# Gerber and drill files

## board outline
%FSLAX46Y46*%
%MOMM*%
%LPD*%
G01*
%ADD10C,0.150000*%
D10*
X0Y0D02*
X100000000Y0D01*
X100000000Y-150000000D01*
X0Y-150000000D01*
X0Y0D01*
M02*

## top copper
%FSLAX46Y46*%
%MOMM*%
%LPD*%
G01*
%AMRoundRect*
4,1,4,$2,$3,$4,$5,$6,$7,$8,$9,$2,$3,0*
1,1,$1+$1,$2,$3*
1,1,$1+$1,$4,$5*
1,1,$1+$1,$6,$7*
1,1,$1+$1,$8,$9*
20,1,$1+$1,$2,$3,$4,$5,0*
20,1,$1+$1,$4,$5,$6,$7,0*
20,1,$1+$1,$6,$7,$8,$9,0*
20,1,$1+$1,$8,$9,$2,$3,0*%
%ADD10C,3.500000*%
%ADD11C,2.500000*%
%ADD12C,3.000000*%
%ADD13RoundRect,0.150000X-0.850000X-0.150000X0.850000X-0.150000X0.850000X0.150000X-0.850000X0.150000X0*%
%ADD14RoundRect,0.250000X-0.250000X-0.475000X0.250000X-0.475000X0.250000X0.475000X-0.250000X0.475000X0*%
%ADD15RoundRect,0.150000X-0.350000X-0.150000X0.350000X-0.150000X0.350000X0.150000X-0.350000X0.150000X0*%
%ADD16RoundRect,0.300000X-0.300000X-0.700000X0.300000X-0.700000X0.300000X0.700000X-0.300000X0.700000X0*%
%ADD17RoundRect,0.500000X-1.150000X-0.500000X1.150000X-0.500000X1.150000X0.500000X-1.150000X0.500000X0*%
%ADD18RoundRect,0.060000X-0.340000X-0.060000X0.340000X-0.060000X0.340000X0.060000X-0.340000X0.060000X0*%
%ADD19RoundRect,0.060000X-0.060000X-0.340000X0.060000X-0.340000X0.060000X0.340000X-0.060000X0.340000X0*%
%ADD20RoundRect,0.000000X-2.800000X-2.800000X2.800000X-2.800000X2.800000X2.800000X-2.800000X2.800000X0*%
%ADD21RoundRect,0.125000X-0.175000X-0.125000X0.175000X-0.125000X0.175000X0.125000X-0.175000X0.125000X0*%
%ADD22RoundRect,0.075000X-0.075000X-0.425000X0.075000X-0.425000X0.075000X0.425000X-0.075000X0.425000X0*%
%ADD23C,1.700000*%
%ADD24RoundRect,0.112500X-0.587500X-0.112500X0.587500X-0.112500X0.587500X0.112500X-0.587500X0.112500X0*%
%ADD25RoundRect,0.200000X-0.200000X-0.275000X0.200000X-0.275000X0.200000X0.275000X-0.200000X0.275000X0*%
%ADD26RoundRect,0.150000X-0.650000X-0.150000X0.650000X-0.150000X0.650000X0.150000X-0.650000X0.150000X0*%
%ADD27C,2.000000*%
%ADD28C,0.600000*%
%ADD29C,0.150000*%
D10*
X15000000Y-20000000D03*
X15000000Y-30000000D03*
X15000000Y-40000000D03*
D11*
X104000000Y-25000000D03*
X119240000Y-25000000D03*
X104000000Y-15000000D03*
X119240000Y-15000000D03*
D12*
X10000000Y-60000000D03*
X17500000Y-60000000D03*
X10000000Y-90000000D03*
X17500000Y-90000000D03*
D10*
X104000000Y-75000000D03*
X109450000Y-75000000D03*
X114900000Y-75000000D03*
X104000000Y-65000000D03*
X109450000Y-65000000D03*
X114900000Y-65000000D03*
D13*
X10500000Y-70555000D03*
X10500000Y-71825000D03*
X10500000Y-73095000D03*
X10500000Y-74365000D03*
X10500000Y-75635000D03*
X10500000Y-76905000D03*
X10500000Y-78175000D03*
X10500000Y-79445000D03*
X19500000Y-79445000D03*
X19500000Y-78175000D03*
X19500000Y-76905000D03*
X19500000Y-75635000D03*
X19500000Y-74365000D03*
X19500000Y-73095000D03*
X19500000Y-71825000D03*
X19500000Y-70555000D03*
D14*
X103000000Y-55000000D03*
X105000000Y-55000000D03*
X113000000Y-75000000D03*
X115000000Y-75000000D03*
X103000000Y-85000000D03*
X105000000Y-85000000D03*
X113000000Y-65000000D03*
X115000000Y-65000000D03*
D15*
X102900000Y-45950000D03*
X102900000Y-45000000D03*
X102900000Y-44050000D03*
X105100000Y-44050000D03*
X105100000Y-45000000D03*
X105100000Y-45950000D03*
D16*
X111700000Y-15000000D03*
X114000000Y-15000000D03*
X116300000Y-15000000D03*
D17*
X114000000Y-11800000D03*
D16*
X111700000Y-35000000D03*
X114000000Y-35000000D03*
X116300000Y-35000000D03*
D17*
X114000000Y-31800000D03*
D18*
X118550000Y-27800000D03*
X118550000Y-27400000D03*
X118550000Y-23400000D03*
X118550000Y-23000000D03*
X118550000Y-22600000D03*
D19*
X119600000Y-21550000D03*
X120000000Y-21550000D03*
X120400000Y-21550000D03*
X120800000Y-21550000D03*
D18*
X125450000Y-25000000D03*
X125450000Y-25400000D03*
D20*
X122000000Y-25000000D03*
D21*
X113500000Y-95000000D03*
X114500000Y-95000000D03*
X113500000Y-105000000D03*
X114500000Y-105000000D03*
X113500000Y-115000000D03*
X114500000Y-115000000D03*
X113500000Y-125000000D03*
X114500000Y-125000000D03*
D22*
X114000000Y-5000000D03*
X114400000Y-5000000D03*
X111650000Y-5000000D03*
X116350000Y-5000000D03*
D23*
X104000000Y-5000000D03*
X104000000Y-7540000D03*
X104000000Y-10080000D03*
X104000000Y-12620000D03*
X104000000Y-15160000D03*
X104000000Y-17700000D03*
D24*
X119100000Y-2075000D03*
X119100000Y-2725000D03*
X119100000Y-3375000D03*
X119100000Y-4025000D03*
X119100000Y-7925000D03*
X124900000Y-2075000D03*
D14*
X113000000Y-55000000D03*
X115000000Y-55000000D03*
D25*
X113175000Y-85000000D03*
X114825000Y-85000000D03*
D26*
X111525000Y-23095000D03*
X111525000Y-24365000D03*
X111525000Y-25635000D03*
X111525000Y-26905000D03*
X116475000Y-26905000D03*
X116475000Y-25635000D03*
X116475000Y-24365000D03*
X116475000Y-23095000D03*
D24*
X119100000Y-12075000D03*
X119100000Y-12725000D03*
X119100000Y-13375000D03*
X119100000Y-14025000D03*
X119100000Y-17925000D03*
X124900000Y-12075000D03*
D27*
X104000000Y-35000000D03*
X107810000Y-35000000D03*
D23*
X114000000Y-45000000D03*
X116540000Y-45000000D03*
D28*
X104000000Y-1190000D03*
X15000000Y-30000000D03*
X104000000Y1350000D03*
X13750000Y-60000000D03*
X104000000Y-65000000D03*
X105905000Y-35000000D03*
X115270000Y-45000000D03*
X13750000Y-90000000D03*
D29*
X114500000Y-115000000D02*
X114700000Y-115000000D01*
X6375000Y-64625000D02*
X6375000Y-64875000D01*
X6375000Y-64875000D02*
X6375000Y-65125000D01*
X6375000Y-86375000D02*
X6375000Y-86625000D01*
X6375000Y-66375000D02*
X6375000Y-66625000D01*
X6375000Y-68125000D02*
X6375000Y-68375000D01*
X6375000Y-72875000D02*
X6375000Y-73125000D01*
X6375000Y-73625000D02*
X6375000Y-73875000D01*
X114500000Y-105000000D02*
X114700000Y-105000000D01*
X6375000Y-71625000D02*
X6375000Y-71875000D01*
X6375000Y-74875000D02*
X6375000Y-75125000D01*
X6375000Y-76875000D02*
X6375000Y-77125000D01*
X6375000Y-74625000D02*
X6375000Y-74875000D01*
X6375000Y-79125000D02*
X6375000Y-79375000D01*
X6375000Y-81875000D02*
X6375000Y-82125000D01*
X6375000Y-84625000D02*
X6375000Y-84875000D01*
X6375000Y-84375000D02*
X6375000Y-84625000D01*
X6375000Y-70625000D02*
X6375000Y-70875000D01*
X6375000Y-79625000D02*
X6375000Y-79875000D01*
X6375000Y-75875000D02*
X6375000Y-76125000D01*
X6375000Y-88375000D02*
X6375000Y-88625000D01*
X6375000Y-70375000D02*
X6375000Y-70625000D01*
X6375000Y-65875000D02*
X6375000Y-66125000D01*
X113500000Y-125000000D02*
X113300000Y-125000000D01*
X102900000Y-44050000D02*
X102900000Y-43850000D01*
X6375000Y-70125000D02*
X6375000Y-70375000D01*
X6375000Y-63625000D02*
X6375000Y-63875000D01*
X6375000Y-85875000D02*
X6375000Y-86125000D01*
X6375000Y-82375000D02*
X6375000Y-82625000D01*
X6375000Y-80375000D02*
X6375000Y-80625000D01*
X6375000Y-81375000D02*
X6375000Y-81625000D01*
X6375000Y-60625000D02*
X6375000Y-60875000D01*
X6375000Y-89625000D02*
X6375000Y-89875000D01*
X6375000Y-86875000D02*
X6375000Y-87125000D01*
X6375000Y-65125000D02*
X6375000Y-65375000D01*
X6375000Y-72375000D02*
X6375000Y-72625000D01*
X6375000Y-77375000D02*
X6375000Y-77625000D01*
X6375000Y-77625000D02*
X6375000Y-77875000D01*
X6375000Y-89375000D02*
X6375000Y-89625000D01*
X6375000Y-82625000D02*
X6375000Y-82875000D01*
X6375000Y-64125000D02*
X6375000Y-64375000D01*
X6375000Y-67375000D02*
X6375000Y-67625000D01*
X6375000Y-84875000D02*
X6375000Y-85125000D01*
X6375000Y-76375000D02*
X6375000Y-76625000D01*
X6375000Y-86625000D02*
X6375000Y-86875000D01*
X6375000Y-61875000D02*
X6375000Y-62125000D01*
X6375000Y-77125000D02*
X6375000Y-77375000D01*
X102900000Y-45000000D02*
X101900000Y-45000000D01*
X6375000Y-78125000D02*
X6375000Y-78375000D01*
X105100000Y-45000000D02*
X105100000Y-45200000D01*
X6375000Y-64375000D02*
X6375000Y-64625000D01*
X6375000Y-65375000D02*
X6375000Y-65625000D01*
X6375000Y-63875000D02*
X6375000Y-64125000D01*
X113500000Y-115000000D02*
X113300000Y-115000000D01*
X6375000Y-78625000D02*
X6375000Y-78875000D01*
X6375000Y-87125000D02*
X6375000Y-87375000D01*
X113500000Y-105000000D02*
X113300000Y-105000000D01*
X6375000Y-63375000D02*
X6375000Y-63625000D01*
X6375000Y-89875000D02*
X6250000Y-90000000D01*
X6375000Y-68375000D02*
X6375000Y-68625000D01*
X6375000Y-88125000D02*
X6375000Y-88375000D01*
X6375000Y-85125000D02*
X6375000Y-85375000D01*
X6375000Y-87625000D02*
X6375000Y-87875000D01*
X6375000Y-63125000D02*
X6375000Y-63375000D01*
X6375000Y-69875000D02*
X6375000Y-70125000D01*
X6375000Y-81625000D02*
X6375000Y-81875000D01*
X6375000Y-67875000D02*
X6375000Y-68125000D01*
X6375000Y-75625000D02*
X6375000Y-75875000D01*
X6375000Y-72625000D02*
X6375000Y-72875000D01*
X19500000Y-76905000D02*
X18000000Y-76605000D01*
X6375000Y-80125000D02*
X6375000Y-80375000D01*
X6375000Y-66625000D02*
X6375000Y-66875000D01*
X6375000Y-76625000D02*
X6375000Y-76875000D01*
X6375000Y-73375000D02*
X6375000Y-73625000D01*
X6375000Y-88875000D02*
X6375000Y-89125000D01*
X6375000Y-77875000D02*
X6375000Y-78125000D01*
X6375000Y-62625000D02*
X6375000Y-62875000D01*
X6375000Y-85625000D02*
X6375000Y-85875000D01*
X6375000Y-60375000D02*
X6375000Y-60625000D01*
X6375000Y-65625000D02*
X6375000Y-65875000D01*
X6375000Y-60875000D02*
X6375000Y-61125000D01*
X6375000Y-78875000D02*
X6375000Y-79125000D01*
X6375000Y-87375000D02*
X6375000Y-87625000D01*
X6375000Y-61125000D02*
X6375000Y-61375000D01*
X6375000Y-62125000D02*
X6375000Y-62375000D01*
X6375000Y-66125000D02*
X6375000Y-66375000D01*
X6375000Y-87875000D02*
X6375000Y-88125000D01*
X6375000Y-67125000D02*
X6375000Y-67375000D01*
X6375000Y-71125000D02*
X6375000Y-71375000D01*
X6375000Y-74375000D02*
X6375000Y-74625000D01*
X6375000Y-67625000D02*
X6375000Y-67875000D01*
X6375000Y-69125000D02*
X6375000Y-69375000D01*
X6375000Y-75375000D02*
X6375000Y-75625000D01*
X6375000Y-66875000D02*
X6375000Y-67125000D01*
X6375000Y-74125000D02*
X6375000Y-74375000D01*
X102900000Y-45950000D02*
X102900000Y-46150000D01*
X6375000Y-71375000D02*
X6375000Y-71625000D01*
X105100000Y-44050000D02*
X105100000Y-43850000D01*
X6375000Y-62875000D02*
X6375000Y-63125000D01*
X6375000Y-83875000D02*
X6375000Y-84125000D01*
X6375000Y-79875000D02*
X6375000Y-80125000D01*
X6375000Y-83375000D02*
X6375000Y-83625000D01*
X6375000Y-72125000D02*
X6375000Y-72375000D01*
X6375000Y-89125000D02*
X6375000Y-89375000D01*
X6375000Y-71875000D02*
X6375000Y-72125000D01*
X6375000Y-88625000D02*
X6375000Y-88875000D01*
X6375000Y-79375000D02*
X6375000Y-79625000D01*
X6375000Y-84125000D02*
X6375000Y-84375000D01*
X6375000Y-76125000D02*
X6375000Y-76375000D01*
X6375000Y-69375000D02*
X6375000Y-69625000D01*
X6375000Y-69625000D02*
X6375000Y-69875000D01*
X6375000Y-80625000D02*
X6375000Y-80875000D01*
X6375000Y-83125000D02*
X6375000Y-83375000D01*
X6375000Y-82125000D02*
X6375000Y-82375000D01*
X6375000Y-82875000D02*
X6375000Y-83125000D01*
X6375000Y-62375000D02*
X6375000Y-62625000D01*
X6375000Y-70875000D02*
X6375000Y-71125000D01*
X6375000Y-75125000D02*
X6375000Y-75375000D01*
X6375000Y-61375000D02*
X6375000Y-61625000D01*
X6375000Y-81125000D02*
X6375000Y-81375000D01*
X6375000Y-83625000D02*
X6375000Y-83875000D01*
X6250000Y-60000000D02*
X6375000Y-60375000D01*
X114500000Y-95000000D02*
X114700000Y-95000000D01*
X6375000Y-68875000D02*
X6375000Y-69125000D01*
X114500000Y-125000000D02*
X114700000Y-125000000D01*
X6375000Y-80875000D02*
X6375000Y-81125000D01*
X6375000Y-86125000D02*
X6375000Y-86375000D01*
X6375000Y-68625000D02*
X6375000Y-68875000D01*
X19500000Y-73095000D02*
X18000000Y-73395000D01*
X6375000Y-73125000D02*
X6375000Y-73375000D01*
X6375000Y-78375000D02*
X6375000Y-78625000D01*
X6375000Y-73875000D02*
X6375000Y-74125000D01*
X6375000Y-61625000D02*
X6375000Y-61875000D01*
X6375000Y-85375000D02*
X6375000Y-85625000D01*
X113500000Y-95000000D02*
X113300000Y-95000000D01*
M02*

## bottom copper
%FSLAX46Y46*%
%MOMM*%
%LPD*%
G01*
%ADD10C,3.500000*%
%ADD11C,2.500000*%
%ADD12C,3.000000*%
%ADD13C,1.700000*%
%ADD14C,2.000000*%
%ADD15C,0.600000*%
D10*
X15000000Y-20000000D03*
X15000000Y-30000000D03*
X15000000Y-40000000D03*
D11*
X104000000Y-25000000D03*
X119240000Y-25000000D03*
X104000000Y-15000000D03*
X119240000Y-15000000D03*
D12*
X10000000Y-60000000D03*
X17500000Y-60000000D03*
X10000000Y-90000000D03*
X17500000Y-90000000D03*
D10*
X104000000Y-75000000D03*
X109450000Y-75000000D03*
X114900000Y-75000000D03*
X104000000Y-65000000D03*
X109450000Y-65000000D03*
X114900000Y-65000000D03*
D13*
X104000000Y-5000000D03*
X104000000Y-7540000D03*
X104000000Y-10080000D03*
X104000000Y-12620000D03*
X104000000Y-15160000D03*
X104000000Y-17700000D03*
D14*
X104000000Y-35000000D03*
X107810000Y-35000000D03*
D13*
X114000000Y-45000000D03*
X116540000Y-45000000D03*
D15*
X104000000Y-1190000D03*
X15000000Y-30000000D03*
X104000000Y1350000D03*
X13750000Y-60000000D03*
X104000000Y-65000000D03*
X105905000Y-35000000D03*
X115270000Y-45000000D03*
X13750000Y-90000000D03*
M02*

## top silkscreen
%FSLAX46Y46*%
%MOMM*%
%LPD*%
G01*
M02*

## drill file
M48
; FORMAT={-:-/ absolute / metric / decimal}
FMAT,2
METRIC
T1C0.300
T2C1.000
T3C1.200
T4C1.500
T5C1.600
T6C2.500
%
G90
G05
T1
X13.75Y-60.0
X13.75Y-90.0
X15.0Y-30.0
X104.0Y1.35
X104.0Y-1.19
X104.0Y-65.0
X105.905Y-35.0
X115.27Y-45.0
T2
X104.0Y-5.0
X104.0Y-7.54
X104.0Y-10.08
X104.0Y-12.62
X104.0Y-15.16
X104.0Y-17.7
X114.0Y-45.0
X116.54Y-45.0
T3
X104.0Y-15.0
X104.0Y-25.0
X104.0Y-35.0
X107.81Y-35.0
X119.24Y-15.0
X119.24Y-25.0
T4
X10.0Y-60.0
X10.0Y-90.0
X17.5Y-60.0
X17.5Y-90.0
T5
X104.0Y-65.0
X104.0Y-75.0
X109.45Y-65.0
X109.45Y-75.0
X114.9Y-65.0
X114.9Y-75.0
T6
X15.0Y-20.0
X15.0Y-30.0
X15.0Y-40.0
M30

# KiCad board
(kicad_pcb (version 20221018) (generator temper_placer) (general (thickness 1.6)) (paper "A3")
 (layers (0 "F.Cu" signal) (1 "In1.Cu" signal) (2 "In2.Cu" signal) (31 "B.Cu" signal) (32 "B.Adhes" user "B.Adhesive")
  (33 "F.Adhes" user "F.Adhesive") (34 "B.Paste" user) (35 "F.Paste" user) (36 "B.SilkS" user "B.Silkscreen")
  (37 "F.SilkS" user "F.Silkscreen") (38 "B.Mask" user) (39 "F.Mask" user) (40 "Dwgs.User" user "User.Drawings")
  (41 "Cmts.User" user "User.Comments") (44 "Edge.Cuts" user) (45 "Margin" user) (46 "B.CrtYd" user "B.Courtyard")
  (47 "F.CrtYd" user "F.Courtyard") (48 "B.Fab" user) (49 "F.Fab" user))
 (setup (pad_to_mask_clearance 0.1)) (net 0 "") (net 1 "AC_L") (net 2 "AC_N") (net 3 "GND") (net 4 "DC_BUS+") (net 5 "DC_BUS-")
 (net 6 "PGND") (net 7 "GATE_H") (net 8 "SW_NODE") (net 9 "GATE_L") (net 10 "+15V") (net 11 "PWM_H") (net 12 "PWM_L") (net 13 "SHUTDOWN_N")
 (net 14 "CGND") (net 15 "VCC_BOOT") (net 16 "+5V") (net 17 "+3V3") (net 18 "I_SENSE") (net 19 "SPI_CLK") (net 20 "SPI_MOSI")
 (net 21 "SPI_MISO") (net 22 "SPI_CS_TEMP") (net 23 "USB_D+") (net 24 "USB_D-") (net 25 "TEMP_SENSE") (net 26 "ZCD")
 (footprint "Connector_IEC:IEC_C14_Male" (layer "F.Cu") (at 15 20 0) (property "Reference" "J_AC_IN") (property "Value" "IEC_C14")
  (pad "1" thru_hole circle (at 0 0) (size 3.5 3.5) (drill 2.5) (layers *.Cu *.Mask) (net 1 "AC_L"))
  (pad "2" thru_hole circle (at 0 10) (size 3.5 3.5) (drill 2.5) (layers *.Cu *.Mask) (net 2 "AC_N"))
  (pad "3" thru_hole circle (at 0 20) (size 3.5 3.5) (drill 2.5) (layers *.Cu *.Mask) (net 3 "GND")))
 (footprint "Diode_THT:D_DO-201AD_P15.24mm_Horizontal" (layer "F.Cu") (at 104 25 0) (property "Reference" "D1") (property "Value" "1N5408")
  (pad "1" thru_hole circle (at 0 0) (size 2.5 2.5) (drill 1.2) (layers *.Cu *.Mask) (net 1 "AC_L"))
  (pad "2" thru_hole circle (at 15.24 0) (size 2.5 2.5) (drill 1.2) (layers *.Cu *.Mask) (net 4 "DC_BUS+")))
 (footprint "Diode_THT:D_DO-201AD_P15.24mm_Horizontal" (layer "F.Cu") (at 104 15 0) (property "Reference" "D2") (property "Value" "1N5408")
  (pad "1" thru_hole circle (at 0 0) (size 2.5 2.5) (drill 1.2) (layers *.Cu *.Mask) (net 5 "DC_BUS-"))
  (pad "2" thru_hole circle (at 15.24 0) (size 2.5 2.5) (drill 1.2) (layers *.Cu *.Mask) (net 2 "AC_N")))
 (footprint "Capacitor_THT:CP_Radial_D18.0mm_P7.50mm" (layer "F.Cu") (at 10 60 0) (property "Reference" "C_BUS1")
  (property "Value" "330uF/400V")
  (pad "1" thru_hole circle (at 0 0) (size 3 3) (drill 1.5) (layers *.Cu *.Mask) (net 4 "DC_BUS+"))
  (pad "2" thru_hole circle (at 7.5 0) (size 3 3) (drill 1.5) (layers *.Cu *.Mask) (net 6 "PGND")))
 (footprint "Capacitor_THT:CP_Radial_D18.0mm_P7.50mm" (layer "F.Cu") (at 10 90 0) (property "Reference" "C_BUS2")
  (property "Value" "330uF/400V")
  (pad "1" thru_hole circle (at 0 0) (size 3 3) (drill 1.5) (layers *.Cu *.Mask) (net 4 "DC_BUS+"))
  (pad "2" thru_hole circle (at 7.5 0) (size 3 3) (drill 1.5) (layers *.Cu *.Mask) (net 6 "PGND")))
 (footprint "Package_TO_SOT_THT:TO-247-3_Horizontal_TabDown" (layer "F.Cu") (at 104 75 0) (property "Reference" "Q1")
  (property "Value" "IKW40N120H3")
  (pad "1" thru_hole circle (at 0 0) (size 3.5 3.5) (drill 1.6) (layers *.Cu *.Mask) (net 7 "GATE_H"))
  (pad "2" thru_hole circle (at 5.45 0) (size 3.5 3.5) (drill 1.6) (layers *.Cu *.Mask) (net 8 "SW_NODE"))
  (pad "3" thru_hole circle (at 10.9 0) (size 3.5 3.5) (drill 1.6) (layers *.Cu *.Mask) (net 4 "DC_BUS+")))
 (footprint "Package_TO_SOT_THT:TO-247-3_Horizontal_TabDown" (layer "F.Cu") (at 104 65 0) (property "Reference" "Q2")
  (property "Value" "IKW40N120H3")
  (pad "1" thru_hole circle (at 0 0) (size 3.5 3.5) (drill 1.6) (layers *.Cu *.Mask) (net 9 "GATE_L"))
  (pad "2" thru_hole circle (at 5.45 0) (size 3.5 3.5) (drill 1.6) (layers *.Cu *.Mask) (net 6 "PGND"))
  (pad "3" thru_hole circle (at 10.9 0) (size 3.5 3.5) (drill 1.6) (layers *.Cu *.Mask) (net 8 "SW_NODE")))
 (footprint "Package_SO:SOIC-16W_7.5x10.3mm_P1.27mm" (layer "F.Cu") (at 15 75 0) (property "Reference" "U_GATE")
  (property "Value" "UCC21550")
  (pad "1" smd roundrect (at -4.5 -4.445) (size 2 0.6) (layers "F.Cu" "F.Paste" "F.Mask") (roundrect_rratio 0.25) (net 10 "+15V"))
  (pad "2" smd roundrect (at -4.5 -3.175) (size 2 0.6) (layers "F.Cu" "F.Paste" "F.Mask") (roundrect_rratio 0.25) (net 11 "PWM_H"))
  (pad "3" smd roundrect (at -4.5 -1.905) (size 2 0.6) (layers "F.Cu" "F.Paste" "F.Mask") (roundrect_rratio 0.25) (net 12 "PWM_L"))
  (pad "4" smd roundrect (at -4.5 -0.635) (size 2 0.6) (layers "F.Cu" "F.Paste" "F.Mask") (roundrect_rratio 0.25) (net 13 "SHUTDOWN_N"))
  (pad "5" smd roundrect (at -4.5 0.635) (size 2 0.6) (layers "F.Cu" "F.Paste" "F.Mask") (roundrect_rratio 0.25) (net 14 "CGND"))
  (pad "6" smd roundrect (at -4.5 1.905) (size 2 0.6) (layers "F.Cu" "F.Paste" "F.Mask") (roundrect_rratio 0.25) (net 14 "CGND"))
  (pad "7" smd roundrect (at -4.5 3.175) (size 2 0.6) (layers "F.Cu" "F.Paste" "F.Mask") (roundrect_rratio 0.25) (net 14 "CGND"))
  (pad "8" smd roundrect (at -4.5 4.445) (size 2 0.6) (layers "F.Cu" "F.Paste" "F.Mask") (roundrect_rratio 0.25) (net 14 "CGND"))
  (pad "9" smd roundrect (at 4.5 4.445) (size 2 0.6) (layers "F.Cu" "F.Paste" "F.Mask") (roundrect_rratio 0.25) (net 8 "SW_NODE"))
  (pad "10" smd roundrect (at 4.5 3.175) (size 2 0.6) (layers "F.Cu" "F.Paste" "F.Mask") (roundrect_rratio 0.25) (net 9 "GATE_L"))
  (pad "11" smd roundrect (at 4.5 1.905) (size 2 0.6) (layers "F.Cu" "F.Paste" "F.Mask") (roundrect_rratio 0.25) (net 10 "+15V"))
  (pad "12" smd roundrect (at 4.5 0.635) (size 2 0.6) (layers "F.Cu" "F.Paste" "F.Mask") (roundrect_rratio 0.25) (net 6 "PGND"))
  (pad "13" smd roundrect (at 4.5 -0.635) (size 2 0.6) (layers "F.Cu" "F.Paste" "F.Mask") (roundrect_rratio 0.25) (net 6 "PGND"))
  (pad "14" smd roundrect (at 4.5 -1.905) (size 2 0.6) (layers "F.Cu" "F.Paste" "F.Mask") (roundrect_rratio 0.25) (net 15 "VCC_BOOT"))
  (pad "15" smd roundrect (at 4.5 -3.175) (size 2 0.6) (layers "F.Cu" "F.Paste" "F.Mask") (roundrect_rratio 0.25) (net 7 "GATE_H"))
  (pad "16" smd roundrect (at 4.5 -4.445) (size 2 0.6) (layers "F.Cu" "F.Paste" "F.Mask") (roundrect_rratio 0.25) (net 8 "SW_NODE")))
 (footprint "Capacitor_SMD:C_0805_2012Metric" (layer "F.Cu") (at 104 55 0) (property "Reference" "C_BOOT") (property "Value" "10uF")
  (pad "1" smd roundrect (at -1 0) (size 1 1.45) (layers "F.Cu" "F.Paste" "F.Mask") (roundrect_rratio 0.25) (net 15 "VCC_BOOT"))
  (pad "2" smd roundrect (at 1 0) (size 1 1.45) (layers "F.Cu" "F.Paste" "F.Mask") (roundrect_rratio 0.25) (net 8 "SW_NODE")))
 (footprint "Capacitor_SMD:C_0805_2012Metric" (layer "F.Cu") (at 114 75 0) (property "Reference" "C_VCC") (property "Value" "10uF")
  (pad "1" smd roundrect (at -1 0) (size 1 1.45) (layers "F.Cu" "F.Paste" "F.Mask") (roundrect_rratio 0.25) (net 10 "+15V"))
  (pad "2" smd roundrect (at 1 0) (size 1 1.45) (layers "F.Cu" "F.Paste" "F.Mask") (roundrect_rratio 0.25) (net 14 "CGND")))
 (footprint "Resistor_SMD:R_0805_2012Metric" (layer "F.Cu") (at 104 85 0) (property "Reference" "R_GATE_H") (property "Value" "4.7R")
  (pad "1" smd roundrect (at -1 0) (size 1 1.45) (layers "F.Cu" "F.Paste" "F.Mask") (roundrect_rratio 0.25) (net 7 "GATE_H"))
  (pad "2" smd roundrect (at 1 0) (size 1 1.45) (layers "F.Cu" "F.Paste" "F.Mask") (roundrect_rratio 0.25) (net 7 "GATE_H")))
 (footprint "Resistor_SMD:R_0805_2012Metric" (layer "F.Cu") (at 114 65 0) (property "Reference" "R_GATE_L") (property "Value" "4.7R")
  (pad "1" smd roundrect (at -1 0) (size 1 1.45) (layers "F.Cu" "F.Paste" "F.Mask") (roundrect_rratio 0.25) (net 9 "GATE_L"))
  (pad "2" smd roundrect (at 1 0) (size 1 1.45) (layers "F.Cu" "F.Paste" "F.Mask") (roundrect_rratio 0.25) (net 9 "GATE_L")))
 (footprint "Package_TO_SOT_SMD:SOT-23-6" (layer "F.Cu") (at 104 45 0) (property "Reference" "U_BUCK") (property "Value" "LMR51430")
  (pad "1" smd roundrect (at -1.1 0.95) (size 1 0.6) (layers "F.Cu" "F.Paste" "F.Mask") (roundrect_rratio 0.25) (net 3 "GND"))
  (pad "2" smd roundrect (at -1.1 0) (size 1 0.6) (layers "F.Cu" "F.Paste" "F.Mask") (roundrect_rratio 0.25) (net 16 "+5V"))
  (pad "3" smd roundrect (at -1.1 -0.95) (size 1 0.6) (layers "F.Cu" "F.Paste" "F.Mask") (roundrect_rratio 0.25) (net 10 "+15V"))
  (pad "4" smd roundrect (at 1.1 -0.95) (size 1 0.6) (layers "F.Cu" "F.Paste" "F.Mask") (roundrect_rratio 0.25) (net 16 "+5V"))
  (pad "5" smd roundrect (at 1.1 0) (size 1 0.6) (layers "F.Cu" "F.Paste" "F.Mask") (roundrect_rratio 0.25) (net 3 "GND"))
  (pad "6" smd roundrect (at 1.1 0.95) (size 1 0.6) (layers "F.Cu" "F.Paste" "F.Mask") (roundrect_rratio 0.25) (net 3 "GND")))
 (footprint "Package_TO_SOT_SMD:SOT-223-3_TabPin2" (layer "F.Cu") (at 114 15 0) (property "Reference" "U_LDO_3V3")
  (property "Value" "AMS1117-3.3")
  (pad "1" smd roundrect (at -2.3 0) (size 1.2 2) (layers "F.Cu" "F.Paste" "F.Mask") (roundrect_rratio 0.25) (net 3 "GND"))
  (pad "2" smd roundrect (at 0 0) (size 1.2 2) (layers "F.Cu" "F.Paste" "F.Mask") (roundrect_rratio 0.25) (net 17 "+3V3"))
  (pad "3" smd roundrect (at 2.3 0) (size 1.2 2) (layers "F.Cu" "F.Paste" "F.Mask") (roundrect_rratio 0.25) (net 16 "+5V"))
  (pad "4" smd roundrect (at 0 -3.2) (size 3.3 2) (layers "F.Cu" "F.Paste" "F.Mask") (roundrect_rratio 0.25) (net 17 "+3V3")))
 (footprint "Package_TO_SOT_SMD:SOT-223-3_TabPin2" (layer "F.Cu") (at 114 35 0) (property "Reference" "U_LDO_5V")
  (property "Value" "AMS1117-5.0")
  (pad "1" smd roundrect (at -2.3 0) (size 1.2 2) (layers "F.Cu" "F.Paste" "F.Mask") (roundrect_rratio 0.25) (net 3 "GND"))
  (pad "2" smd roundrect (at 0 0) (size 1.2 2) (layers "F.Cu" "F.Paste" "F.Mask") (roundrect_rratio 0.25) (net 16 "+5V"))
  (pad "3" smd roundrect (at 2.3 0) (size 1.2 2) (layers "F.Cu" "F.Paste" "F.Mask") (roundrect_rratio 0.25) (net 10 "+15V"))
  (pad "4" smd roundrect (at 0 -3.2) (size 3.3 2) (layers "F.Cu" "F.Paste" "F.Mask") (roundrect_rratio 0.25) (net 16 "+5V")))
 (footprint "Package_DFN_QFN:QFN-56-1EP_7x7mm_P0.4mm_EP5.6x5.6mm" (layer "F.Cu") (at 122 25 0) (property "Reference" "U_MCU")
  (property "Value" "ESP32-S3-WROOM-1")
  (pad "1" smd roundrect (at -3.45 2.8) (size 0.8 0.24) (layers "F.Cu" "F.Paste" "F.Mask") (roundrect_rratio 0.25) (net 17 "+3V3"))
  (pad "2" smd roundrect (at -3.45 2.4) (size 0.8 0.24) (layers "F.Cu" "F.Paste" "F.Mask") (roundrect_rratio 0.25) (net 3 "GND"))
  (pad "13" smd roundrect (at -3.45 -1.6) (size 0.8 0.24) (layers "F.Cu" "F.Paste" "F.Mask") (roundrect_rratio 0.25) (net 11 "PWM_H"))
  (pad "14" smd roundrect (at -3.45 -2) (size 0.8 0.24) (layers "F.Cu" "F.Paste" "F.Mask") (roundrect_rratio 0.25) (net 12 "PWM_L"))
  (pad "15" smd roundrect (at -3.45 -2.4) (size 0.8 0.24) (layers "F.Cu" "F.Paste" "F.Mask") (roundrect_rratio 0.25) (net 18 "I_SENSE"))
  (pad "20" smd roundrect (at -2.4 -3.45) (size 0.24 0.8) (layers "F.Cu" "F.Paste" "F.Mask") (roundrect_rratio 0.25) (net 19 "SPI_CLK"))
  (pad "21" smd roundrect (at -2 -3.45) (size 0.24 0.8) (layers "F.Cu" "F.Paste" "F.Mask") (roundrect_rratio 0.25) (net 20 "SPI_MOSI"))
  (pad "22" smd roundrect (at -1.6 -3.45) (size 0.24 0.8) (layers "F.Cu" "F.Paste" "F.Mask") (roundrect_rratio 0.25) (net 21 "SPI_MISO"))
  (pad "23" smd roundrect (at -1.2 -3.45) (size 0.24 0.8) (layers "F.Cu" "F.Paste" "F.Mask") (roundrect_rratio 0.25) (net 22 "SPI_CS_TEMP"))
  (pad "40" smd roundrect (at 3.45 0) (size 0.8 0.24) (layers "F.Cu" "F.Paste" "F.Mask") (roundrect_rratio 0.25) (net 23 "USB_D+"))
  (pad "41" smd roundrect (at 3.45 0.4) (size 0.8 0.24) (layers "F.Cu" "F.Paste" "F.Mask") (roundrect_rratio 0.25) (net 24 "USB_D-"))
  (pad "57" smd roundrect (at 0 0) (size 5.6 5.6) (layers "F.Cu" "F.Paste" "F.Mask") (roundrect_rratio 0) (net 3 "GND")))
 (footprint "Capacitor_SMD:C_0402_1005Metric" (layer "F.Cu") (at 114 95 0) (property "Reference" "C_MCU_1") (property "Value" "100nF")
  (pad "1" smd roundrect (at -0.5 0) (size 0.6 0.5) (layers "F.Cu" "F.Paste" "F.Mask") (roundrect_rratio 0.25) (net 17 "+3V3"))
  (pad "2" smd roundrect (at 0.5 0) (size 0.6 0.5) (layers "F.Cu" "F.Paste" "F.Mask") (roundrect_rratio 0.25) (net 3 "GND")))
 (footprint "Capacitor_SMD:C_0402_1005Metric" (layer "F.Cu") (at 114 105 0) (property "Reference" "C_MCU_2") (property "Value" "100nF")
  (pad "1" smd roundrect (at -0.5 0) (size 0.6 0.5) (layers "F.Cu" "F.Paste" "F.Mask") (roundrect_rratio 0.25) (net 17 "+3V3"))
  (pad "2" smd roundrect (at 0.5 0) (size 0.6 0.5) (layers "F.Cu" "F.Paste" "F.Mask") (roundrect_rratio 0.25) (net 3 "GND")))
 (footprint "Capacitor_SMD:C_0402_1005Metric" (layer "F.Cu") (at 114 115 0) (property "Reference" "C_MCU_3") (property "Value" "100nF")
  (pad "1" smd roundrect (at -0.5 0) (size 0.6 0.5) (layers "F.Cu" "F.Paste" "F.Mask") (roundrect_rratio 0.25) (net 17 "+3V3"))
  (pad "2" smd roundrect (at 0.5 0) (size 0.6 0.5) (layers "F.Cu" "F.Paste" "F.Mask") (roundrect_rratio 0.25) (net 3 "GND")))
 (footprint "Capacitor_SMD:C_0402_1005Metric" (layer "F.Cu") (at 114 125 0) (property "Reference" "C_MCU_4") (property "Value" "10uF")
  (pad "1" smd roundrect (at -0.5 0) (size 0.6 0.5) (layers "F.Cu" "F.Paste" "F.Mask") (roundrect_rratio 0.25) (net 17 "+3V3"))
  (pad "2" smd roundrect (at 0.5 0) (size 0.6 0.5) (layers "F.Cu" "F.Paste" "F.Mask") (roundrect_rratio 0.25) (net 3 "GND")))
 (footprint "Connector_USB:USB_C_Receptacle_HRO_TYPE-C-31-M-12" (layer "F.Cu") (at 114 5 0) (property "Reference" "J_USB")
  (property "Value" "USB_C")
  (pad "A6" smd roundrect (at 0 0) (size 0.3 1) (layers "F.Cu" "F.Paste" "F.Mask") (roundrect_rratio 0.25) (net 23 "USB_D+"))
  (pad "B6" smd roundrect (at 0.4 0) (size 0.3 1) (layers "F.Cu" "F.Paste" "F.Mask") (roundrect_rratio 0.25) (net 24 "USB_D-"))
  (pad "A1" smd roundrect (at -2.35 0) (size 0.3 1) (layers "F.Cu" "F.Paste" "F.Mask") (roundrect_rratio 0.25) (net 3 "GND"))
  (pad "A12" smd roundrect (at 2.35 0) (size 0.3 1) (layers "F.Cu" "F.Paste" "F.Mask") (roundrect_rratio 0.25) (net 3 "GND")))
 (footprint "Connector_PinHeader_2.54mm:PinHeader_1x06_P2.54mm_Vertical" (layer "F.Cu") (at 104 5 0) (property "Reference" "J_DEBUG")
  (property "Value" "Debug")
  (pad "1" thru_hole circle (at 0 0) (size 1.7 1.7) (drill 1) (layers *.Cu *.Mask) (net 3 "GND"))
  (pad "2" thru_hole circle (at 0 2.54) (size 1.7 1.7) (drill 1) (layers *.Cu *.Mask) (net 17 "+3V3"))
  (pad "3" thru_hole circle (at 0 5.08) (size 1.7 1.7) (drill 1) (layers *.Cu *.Mask) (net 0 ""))
  (pad "4" thru_hole circle (at 0 7.62) (size 1.7 1.7) (drill 1) (layers *.Cu *.Mask) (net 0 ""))
  (pad "5" thru_hole circle (at 0 10.16) (size 1.7 1.7) (drill 1) (layers *.Cu *.Mask) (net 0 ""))
  (pad "6" thru_hole circle (at 0 12.7) (size 1.7 1.7) (drill 1) (layers *.Cu *.Mask) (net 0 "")))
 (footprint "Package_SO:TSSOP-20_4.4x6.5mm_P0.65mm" (layer "F.Cu") (at 122 5 0) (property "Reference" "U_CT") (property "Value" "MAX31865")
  (pad "1" smd roundrect (at -2.9 -2.925) (size 1.4 0.45) (layers "F.Cu" "F.Paste" "F.Mask") (roundrect_rratio 0.25) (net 19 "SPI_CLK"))
  (pad "2" smd roundrect (at -2.9 -2.275) (size 1.4 0.45) (layers "F.Cu" "F.Paste" "F.Mask") (roundrect_rratio 0.25) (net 20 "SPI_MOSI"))
  (pad "3" smd roundrect (at -2.9 -1.625) (size 1.4 0.45) (layers "F.Cu" "F.Paste" "F.Mask") (roundrect_rratio 0.25) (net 21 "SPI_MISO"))
  (pad "4" smd roundrect (at -2.9 -0.975) (size 1.4 0.45) (layers "F.Cu" "F.Paste" "F.Mask") (roundrect_rratio 0.25) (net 22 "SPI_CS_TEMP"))
  (pad "10" smd roundrect (at -2.9 2.925) (size 1.4 0.45) (layers "F.Cu" "F.Paste" "F.Mask") (roundrect_rratio 0.25) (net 3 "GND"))
  (pad "20" smd roundrect (at 2.9 -2.925) (size 1.4 0.45) (layers "F.Cu" "F.Paste" "F.Mask") (roundrect_rratio 0.25) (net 17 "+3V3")))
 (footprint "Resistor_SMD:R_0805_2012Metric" (layer "F.Cu") (at 114 55 0) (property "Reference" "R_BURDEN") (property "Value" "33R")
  (pad "1" smd roundrect (at -1 0) (size 1 1.45) (layers "F.Cu" "F.Paste" "F.Mask") (roundrect_rratio 0.25) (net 18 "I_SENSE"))
  (pad "2" smd roundrect (at 1 0) (size 1 1.45) (layers "F.Cu" "F.Paste" "F.Mask") (roundrect_rratio 0.25) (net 3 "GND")))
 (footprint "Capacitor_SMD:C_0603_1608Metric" (layer "F.Cu") (at 114 85 0) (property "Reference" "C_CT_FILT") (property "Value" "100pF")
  (pad "1" smd roundrect (at -0.825 0) (size 0.8 0.95) (layers "F.Cu" "F.Paste" "F.Mask") (roundrect_rratio 0.25) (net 18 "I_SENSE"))
  (pad "2" smd roundrect (at 0.825 0) (size 0.8 0.95) (layers "F.Cu" "F.Paste" "F.Mask") (roundrect_rratio 0.25) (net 3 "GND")))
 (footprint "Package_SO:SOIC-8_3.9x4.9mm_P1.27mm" (layer "F.Cu") (at 114 25 0) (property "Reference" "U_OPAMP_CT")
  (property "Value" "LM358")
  (pad "1" smd roundrect (at -2.475 -1.905) (size 1.6 0.6) (layers "F.Cu" "F.Paste" "F.Mask") (roundrect_rratio 0.25) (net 18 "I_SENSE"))
  (pad "2" smd roundrect (at -2.475 -0.635) (size 1.6 0.6) (layers "F.Cu" "F.Paste" "F.Mask") (roundrect_rratio 0.25) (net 18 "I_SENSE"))
  (pad "3" smd roundrect (at -2.475 0.635) (size 1.6 0.6) (layers "F.Cu" "F.Paste" "F.Mask") (roundrect_rratio 0.25) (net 18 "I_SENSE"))
  (pad "4" smd roundrect (at -2.475 1.905) (size 1.6 0.6) (layers "F.Cu" "F.Paste" "F.Mask") (roundrect_rratio 0.25) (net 3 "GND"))
  (pad "5" smd roundrect (at 2.475 1.905) (size 1.6 0.6) (layers "F.Cu" "F.Paste" "F.Mask") (roundrect_rratio 0.25) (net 18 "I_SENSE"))
  (pad "6" smd roundrect (at 2.475 0.635) (size 1.6 0.6) (layers "F.Cu" "F.Paste" "F.Mask") (roundrect_rratio 0.25) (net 18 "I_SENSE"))
  (pad "7" smd roundrect (at 2.475 -0.635) (size 1.6 0.6) (layers "F.Cu" "F.Paste" "F.Mask") (roundrect_rratio 0.25) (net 16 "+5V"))
  (pad "8" smd roundrect (at 2.475 -1.905) (size 1.6 0.6) (layers "F.Cu" "F.Paste" "F.Mask") (roundrect_rratio 0.25) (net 16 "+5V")))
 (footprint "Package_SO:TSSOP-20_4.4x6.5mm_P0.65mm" (layer "F.Cu") (at 122 15 0) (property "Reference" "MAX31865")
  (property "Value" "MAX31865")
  (pad "1" smd roundrect (at -2.9 -2.925) (size 1.4 0.45) (layers "F.Cu" "F.Paste" "F.Mask") (roundrect_rratio 0.25) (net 19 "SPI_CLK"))
  (pad "2" smd roundrect (at -2.9 -2.275) (size 1.4 0.45) (layers "F.Cu" "F.Paste" "F.Mask") (roundrect_rratio 0.25) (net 20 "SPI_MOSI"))
  (pad "3" smd roundrect (at -2.9 -1.625) (size 1.4 0.45) (layers "F.Cu" "F.Paste" "F.Mask") (roundrect_rratio 0.25) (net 21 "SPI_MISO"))
  (pad "4" smd roundrect (at -2.9 -0.975) (size 1.4 0.45) (layers "F.Cu" "F.Paste" "F.Mask") (roundrect_rratio 0.25) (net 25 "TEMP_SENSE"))
  (pad "10" smd roundrect (at -2.9 2.925) (size 1.4 0.45) (layers "F.Cu" "F.Paste" "F.Mask") (roundrect_rratio 0.25) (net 3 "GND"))
  (pad "20" smd roundrect (at 2.9 -2.925) (size 1.4 0.45) (layers "F.Cu" "F.Paste" "F.Mask") (roundrect_rratio 0.25) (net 17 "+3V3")))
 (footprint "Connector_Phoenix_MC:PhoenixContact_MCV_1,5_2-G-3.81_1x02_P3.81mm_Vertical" (layer "F.Cu") (at 104 35 0)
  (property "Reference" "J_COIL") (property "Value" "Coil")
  (pad "1" thru_hole circle (at 0 0) (size 2 2) (drill 1.2) (layers *.Cu *.Mask) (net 8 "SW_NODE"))
  (pad "2" thru_hole circle (at 3.81 0) (size 2 2) (drill 1.2) (layers *.Cu *.Mask) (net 3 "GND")))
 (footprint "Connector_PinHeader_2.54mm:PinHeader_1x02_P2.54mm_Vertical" (layer "F.Cu") (at 114 45 0) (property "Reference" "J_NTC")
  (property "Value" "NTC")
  (pad "1" thru_hole circle (at 0 0) (size 1.7 1.7) (drill 1) (layers *.Cu *.Mask) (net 25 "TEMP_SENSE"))
  (pad "2" thru_hole circle (at 2.54 0) (size 1.7 1.7) (drill 1) (layers *.Cu *.Mask) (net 3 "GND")))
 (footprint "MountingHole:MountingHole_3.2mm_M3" (layer "F.Cu") (at 104 95 0) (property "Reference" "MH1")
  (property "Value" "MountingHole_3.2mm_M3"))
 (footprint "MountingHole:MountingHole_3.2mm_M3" (layer "F.Cu") (at 104 105 0) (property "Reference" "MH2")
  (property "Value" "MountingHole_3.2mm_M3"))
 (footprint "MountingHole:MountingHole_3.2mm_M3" (layer "F.Cu") (at 104 115 0) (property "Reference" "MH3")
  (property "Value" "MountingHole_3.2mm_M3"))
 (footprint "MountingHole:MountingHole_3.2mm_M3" (layer "F.Cu") (at 104 125 0) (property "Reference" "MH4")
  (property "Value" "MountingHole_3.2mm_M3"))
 (gr_rect (start 0 0) (end 100 150) (layer "Edge.Cuts") (width 0.15))
 (segment (start 114.5 115.0) (end 114.7 115.0) (width 0.15) (layer "F.Cu") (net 3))
 (segment (start 6.375 64.625) (end 6.375 64.875) (width 0.15) (layer "F.Cu") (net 4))
 (segment (start 6.375 64.875) (end 6.375 65.125) (width 0.15) (layer "F.Cu") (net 4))
 (segment (start 6.375 86.375) (end 6.375 86.625) (width 0.15) (layer "F.Cu") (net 4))
 (segment (start 6.375 66.375) (end 6.375 66.625) (width 0.15) (layer "F.Cu") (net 4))
 (segment (start 6.375 68.125) (end 6.375 68.375) (width 0.15) (layer "F.Cu") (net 4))
 (segment (start 6.375 72.875) (end 6.375 73.125) (width 0.15) (layer "F.Cu") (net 4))
 (segment (start 6.375 73.625) (end 6.375 73.875) (width 0.15) (layer "F.Cu") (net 4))
 (segment (start 114.5 105.0) (end 114.7 105.0) (width 0.15) (layer "F.Cu") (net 3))
 (segment (start 6.375 71.625) (end 6.375 71.875) (width 0.15) (layer "F.Cu") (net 4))
 (segment (start 6.375 74.875) (end 6.375 75.125) (width 0.15) (layer "F.Cu") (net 4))
 (segment (start 6.375 76.875) (end 6.375 77.125) (width 0.15) (layer "F.Cu") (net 4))
 (segment (start 6.375 74.625) (end 6.375 74.875) (width 0.15) (layer "F.Cu") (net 4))
 (segment (start 6.375 79.125) (end 6.375 79.375) (width 0.15) (layer "F.Cu") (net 4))
 (segment (start 6.375 81.875) (end 6.375 82.125) (width 0.15) (layer "F.Cu") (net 4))
 (segment (start 6.375 84.625) (end 6.375 84.875) (width 0.15) (layer "F.Cu") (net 4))
 (segment (start 6.375 84.375) (end 6.375 84.625) (width 0.15) (layer "F.Cu") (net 4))
 (segment (start 6.375 70.625) (end 6.375 70.875) (width 0.15) (layer "F.Cu") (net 4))
 (segment (start 6.375 79.625) (end 6.375 79.875) (width 0.15) (layer "F.Cu") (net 4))
 (segment (start 6.375 75.875) (end 6.375 76.125) (width 0.15) (layer "F.Cu") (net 4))
 (segment (start 6.375 88.375) (end 6.375 88.625) (width 0.15) (layer "F.Cu") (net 4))
 (segment (start 6.375 70.375) (end 6.375 70.625) (width 0.15) (layer "F.Cu") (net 4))
 (segment (start 6.375 65.875) (end 6.375 66.125) (width 0.15) (layer "F.Cu") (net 4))
 (segment (start 113.5 125.0) (end 113.3 125.0) (width 0.15) (layer "F.Cu") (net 17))
 (segment (start 102.9 44.05) (end 102.9 43.849999999999994) (width 0.15) (layer "F.Cu") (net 10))
 (segment (start 6.375 70.125) (end 6.375 70.375) (width 0.15) (layer "F.Cu") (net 4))
 (segment (start 6.375 63.625) (end 6.375 63.875) (width 0.15) (layer "F.Cu") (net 4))
 (segment (start 6.375 85.875) (end 6.375 86.125) (width 0.15) (layer "F.Cu") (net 4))
 (segment (start 6.375 82.375) (end 6.375 82.625) (width 0.15) (layer "F.Cu") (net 4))
 (segment (start 6.375 80.375) (end 6.375 80.625) (width 0.15) (layer "F.Cu") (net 4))
 (segment (start 6.375 81.375) (end 6.375 81.625) (width 0.15) (layer "F.Cu") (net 4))
 (segment (start 6.375 60.625) (end 6.375 60.875) (width 0.15) (layer "F.Cu") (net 4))
 (segment (start 6.375 89.625) (end 6.375 89.875) (width 0.15) (layer "F.Cu") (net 4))
 (segment (start 6.375 86.875) (end 6.375 87.125) (width 0.15) (layer "F.Cu") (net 4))
 (segment (start 6.375 65.125) (end 6.375 65.375) (width 0.15) (layer "F.Cu") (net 4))
 (segment (start 6.375 72.375) (end 6.375 72.625) (width 0.15) (layer "F.Cu") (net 4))
 (segment (start 6.375 77.375) (end 6.375 77.625) (width 0.15) (layer "F.Cu") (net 4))
 (segment (start 6.375 77.625) (end 6.375 77.875) (width 0.15) (layer "F.Cu") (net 4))
 (segment (start 6.375 89.375) (end 6.375 89.625) (width 0.15) (layer "F.Cu") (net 4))
 (segment (start 6.375 82.625) (end 6.375 82.875) (width 0.15) (layer "F.Cu") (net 4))
 (segment (start 6.375 64.125) (end 6.375 64.375) (width 0.15) (layer "F.Cu") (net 4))
 (segment (start 6.375 67.375) (end 6.375 67.625) (width 0.15) (layer "F.Cu") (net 4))
 (segment (start 6.375 84.875) (end 6.375 85.125) (width 0.15) (layer "F.Cu") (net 4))
 (segment (start 6.375 76.375) (end 6.375 76.625) (width 0.15) (layer "F.Cu") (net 4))
 (segment (start 6.375 86.625) (end 6.375 86.875) (width 0.15) (layer "F.Cu") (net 4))
 (segment (start 6.375 61.875) (end 6.375 62.125) (width 0.15) (layer "F.Cu") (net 4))
 (segment (start 6.375 77.125) (end 6.375 77.375) (width 0.15) (layer "F.Cu") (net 4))
 (segment (start 102.9 45.0) (end 101.9 45.0) (width 0.15) (layer "F.Cu") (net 16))
 (segment (start 6.375 78.125) (end 6.375 78.375) (width 0.15) (layer "F.Cu") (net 4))
 (segment (start 105.1 45.0) (end 105.1 45.2) (width 0.15) (layer "F.Cu") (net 3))
 (segment (start 6.375 64.375) (end 6.375 64.625) (width 0.15) (layer "F.Cu") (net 4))
 (segment (start 6.375 65.375) (end 6.375 65.625) (width 0.15) (layer "F.Cu") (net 4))
 (segment (start 6.375 63.875) (end 6.375 64.125) (width 0.15) (layer "F.Cu") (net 4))
 (segment (start 113.5 115.0) (end 113.3 115.0) (width 0.15) (layer "F.Cu") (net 17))
 (segment (start 6.375 78.625) (end 6.375 78.875) (width 0.15) (layer "F.Cu") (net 4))
 (segment (start 6.375 87.125) (end 6.375 87.375) (width 0.15) (layer "F.Cu") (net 4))
 (segment (start 113.5 105.0) (end 113.3 105.0) (width 0.15) (layer "F.Cu") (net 17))
 (segment (start 6.375 63.375) (end 6.375 63.625) (width 0.15) (layer "F.Cu") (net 4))
 (segment (start 6.375 89.875) (end 6.25 90.0) (width 0.15) (layer "F.Cu") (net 4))
 (segment (start 6.375 68.375) (end 6.375 68.625) (width 0.15) (layer "F.Cu") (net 4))
 (segment (start 6.375 88.125) (end 6.375 88.375) (width 0.15) (layer "F.Cu") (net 4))
 (segment (start 6.375 85.125) (end 6.375 85.375) (width 0.15) (layer "F.Cu") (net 4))
 (segment (start 6.375 87.625) (end 6.375 87.875) (width 0.15) (layer "F.Cu") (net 4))
 (segment (start 6.375 63.125) (end 6.375 63.375) (width 0.15) (layer "F.Cu") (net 4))
 (segment (start 6.375 69.875) (end 6.375 70.125) (width 0.15) (layer "F.Cu") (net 4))
 (segment (start 6.375 81.625) (end 6.375 81.875) (width 0.15) (layer "F.Cu") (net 4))
 (segment (start 6.375 67.875) (end 6.375 68.125) (width 0.15) (layer "F.Cu") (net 4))
 (segment (start 6.375 75.625) (end 6.375 75.875) (width 0.15) (layer "F.Cu") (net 4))
 (segment (start 6.375 72.625) (end 6.375 72.875) (width 0.15) (layer "F.Cu") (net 4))
 (segment (start 19.5 76.905) (end 18.0 76.605) (width 0.15) (layer "F.Cu") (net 10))
 (segment (start 6.375 80.125) (end 6.375 80.375) (width 0.15) (layer "F.Cu") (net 4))
 (segment (start 6.375 66.625) (end 6.375 66.875) (width 0.15) (layer "F.Cu") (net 4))
 (segment (start 6.375 76.625) (end 6.375 76.875) (width 0.15) (layer "F.Cu") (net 4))
 (segment (start 6.375 73.375) (end 6.375 73.625) (width 0.15) (layer "F.Cu") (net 4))
 (segment (start 6.375 88.875) (end 6.375 89.125) (width 0.15) (layer "F.Cu") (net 4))
 (segment (start 6.375 77.875) (end 6.375 78.125) (width 0.15) (layer "F.Cu") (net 4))
 (segment (start 6.375 62.625) (end 6.375 62.875) (width 0.15) (layer "F.Cu") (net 4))
 (segment (start 6.375 85.625) (end 6.375 85.875) (width 0.15) (layer "F.Cu") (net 4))
 (segment (start 6.375 60.375) (end 6.375 60.625) (width 0.15) (layer "F.Cu") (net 4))
 (segment (start 6.375 65.625) (end 6.375 65.875) (width 0.15) (layer "F.Cu") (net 4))
 (segment (start 6.375 60.875) (end 6.375 61.125) (width 0.15) (layer "F.Cu") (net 4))
 (segment (start 6.375 78.875) (end 6.375 79.125) (width 0.15) (layer "F.Cu") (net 4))
 (segment (start 6.375 87.375) (end 6.375 87.625) (width 0.15) (layer "F.Cu") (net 4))
 (segment (start 6.375 61.125) (end 6.375 61.375) (width 0.15) (layer "F.Cu") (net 4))
 (segment (start 6.375 62.125) (end 6.375 62.375) (width 0.15) (layer "F.Cu") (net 4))
 (segment (start 6.375 66.125) (end 6.375 66.375) (width 0.15) (layer "F.Cu") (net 4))
 (segment (start 6.375 87.875) (end 6.375 88.125) (width 0.15) (layer "F.Cu") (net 4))
 (segment (start 6.375 67.125) (end 6.375 67.375) (width 0.15) (layer "F.Cu") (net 4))
 (segment (start 6.375 71.125) (end 6.375 71.375) (width 0.15) (layer "F.Cu") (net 4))
 (segment (start 6.375 74.375) (end 6.375 74.625) (width 0.15) (layer "F.Cu") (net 4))
 (segment (start 6.375 67.625) (end 6.375 67.875) (width 0.15) (layer "F.Cu") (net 4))
 (segment (start 6.375 69.125) (end 6.375 69.375) (width 0.15) (layer "F.Cu") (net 4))
 (segment (start 6.375 75.375) (end 6.375 75.625) (width 0.15) (layer "F.Cu") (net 4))
 (segment (start 6.375 66.875) (end 6.375 67.125) (width 0.15) (layer "F.Cu") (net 4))
 (segment (start 6.375 74.125) (end 6.375 74.375) (width 0.15) (layer "F.Cu") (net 4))
 (segment (start 102.9 45.95) (end 102.9 46.150000000000006) (width 0.15) (layer "F.Cu") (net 3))
 (segment (start 6.375 71.375) (end 6.375 71.625) (width 0.15) (layer "F.Cu") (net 4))
 (segment (start 105.1 44.05) (end 105.1 43.849999999999994) (width 0.15) (layer "F.Cu") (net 16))
 (segment (start 6.375 62.875) (end 6.375 63.125) (width 0.15) (layer "F.Cu") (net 4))
 (segment (start 6.375 83.875) (end 6.375 84.125) (width 0.15) (layer "F.Cu") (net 4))
 (segment (start 6.375 79.875) (end 6.375 80.125) (width 0.15) (layer "F.Cu") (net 4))
 (segment (start 6.375 83.375) (end 6.375 83.625) (width 0.15) (layer "F.Cu") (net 4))
 (segment (start 6.375 72.125) (end 6.375 72.375) (width 0.15) (layer "F.Cu") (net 4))
 (segment (start 6.375 89.125) (end 6.375 89.375) (width 0.15) (layer "F.Cu") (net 4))
 (segment (start 6.375 71.875) (end 6.375 72.125) (width 0.15) (layer "F.Cu") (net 4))
 (segment (start 6.375 88.625) (end 6.375 88.875) (width 0.15) (layer "F.Cu") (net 4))
 (segment (start 6.375 79.375) (end 6.375 79.625) (width 0.15) (layer "F.Cu") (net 4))
 (segment (start 6.375 84.125) (end 6.375 84.375) (width 0.15) (layer "F.Cu") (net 4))
 (segment (start 6.375 76.125) (end 6.375 76.375) (width 0.15) (layer "F.Cu") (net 4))
 (segment (start 6.375 69.375) (end 6.375 69.625) (width 0.15) (layer "F.Cu") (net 4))
 (segment (start 6.375 69.625) (end 6.375 69.875) (width 0.15) (layer "F.Cu") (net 4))
 (segment (start 6.375 80.625) (end 6.375 80.875) (width 0.15) (layer "F.Cu") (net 4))
 (segment (start 6.375 83.125) (end 6.375 83.375) (width 0.15) (layer "F.Cu") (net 4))
 (segment (start 6.375 82.125) (end 6.375 82.375) (width 0.15) (layer "F.Cu") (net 4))
 (segment (start 6.375 82.875) (end 6.375 83.125) (width 0.15) (layer "F.Cu") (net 4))
 (segment (start 6.375 62.375) (end 6.375 62.625) (width 0.15) (layer "F.Cu") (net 4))
 (segment (start 6.375 70.875) (end 6.375 71.125) (width 0.15) (layer "F.Cu") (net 4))
 (segment (start 6.375 75.125) (end 6.375 75.375) (width 0.15) (layer "F.Cu") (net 4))
 (segment (start 6.375 61.375) (end 6.375 61.625) (width 0.15) (layer "F.Cu") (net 4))
 (segment (start 6.375 81.125) (end 6.375 81.375) (width 0.15) (layer "F.Cu") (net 4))
 (segment (start 6.375 83.625) (end 6.375 83.875) (width 0.15) (layer "F.Cu") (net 4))
 (segment (start 6.25 60.0) (end 6.375 60.375) (width 0.15) (layer "F.Cu") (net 4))
 (segment (start 114.5 95.0) (end 114.7 95.0) (width 0.15) (layer "F.Cu") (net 3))
 (segment (start 6.375 68.875) (end 6.375 69.125) (width 0.15) (layer "F.Cu") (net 4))
 (segment (start 114.5 125.0) (end 114.7 125.0) (width 0.15) (layer "F.Cu") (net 3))
 (segment (start 6.375 80.875) (end 6.375 81.125) (width 0.15) (layer "F.Cu") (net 4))
 (segment (start 6.375 86.125) (end 6.375 86.375) (width 0.15) (layer "F.Cu") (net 4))
 (segment (start 6.375 68.625) (end 6.375 68.875) (width 0.15) (layer "F.Cu") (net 4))
 (segment (start 19.5 73.095) (end 18.0 73.395) (width 0.15) (layer "F.Cu") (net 15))
 (segment (start 6.375 73.125) (end 6.375 73.375) (width 0.15) (layer "F.Cu") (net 4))
 (segment (start 6.375 78.375) (end 6.375 78.625) (width 0.15) (layer "F.Cu") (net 4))
 (segment (start 6.375 73.875) (end 6.375 74.125) (width 0.15) (layer "F.Cu") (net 4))
 (segment (start 6.375 61.625) (end 6.375 61.875) (width 0.15) (layer "F.Cu") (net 4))
 (segment (start 6.375 85.375) (end 6.375 85.625) (width 0.15) (layer "F.Cu") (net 4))
 (segment (start 113.5 95.0) (end 113.3 95.0) (width 0.15) (layer "F.Cu") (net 17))
 (via (at 104.0 1.1900000000000004) (size 0.6) (drill 0.3) (layers "F.Cu" "In2.Cu") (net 17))
 (via (at 15.0 30.0) (size 0.6) (drill 0.3) (layers "F.Cu" "In1.Cu") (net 3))
 (via (at 104.0 -1.3499999999999996) (size 0.6) (drill 0.3) (layers "F.Cu" "In1.Cu") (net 3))
 (via (at 13.75 60.0) (size 0.6) (drill 0.3) (layers "F.Cu" "In1.Cu") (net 6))
 (via (at 104.0 65.0) (size 0.6) (drill 0.3) (layers "F.Cu" "In1.Cu") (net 6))
 (via (at 105.905 35.0) (size 0.6) (drill 0.3) (layers "F.Cu" "In1.Cu") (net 3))
 (via (at 115.27 45.0) (size 0.6) (drill 0.3) (layers "F.Cu" "In1.Cu") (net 3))
 (via (at 13.75 90.0) (size 0.6) (drill 0.3) (layers "F.Cu" "In1.Cu") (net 6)))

